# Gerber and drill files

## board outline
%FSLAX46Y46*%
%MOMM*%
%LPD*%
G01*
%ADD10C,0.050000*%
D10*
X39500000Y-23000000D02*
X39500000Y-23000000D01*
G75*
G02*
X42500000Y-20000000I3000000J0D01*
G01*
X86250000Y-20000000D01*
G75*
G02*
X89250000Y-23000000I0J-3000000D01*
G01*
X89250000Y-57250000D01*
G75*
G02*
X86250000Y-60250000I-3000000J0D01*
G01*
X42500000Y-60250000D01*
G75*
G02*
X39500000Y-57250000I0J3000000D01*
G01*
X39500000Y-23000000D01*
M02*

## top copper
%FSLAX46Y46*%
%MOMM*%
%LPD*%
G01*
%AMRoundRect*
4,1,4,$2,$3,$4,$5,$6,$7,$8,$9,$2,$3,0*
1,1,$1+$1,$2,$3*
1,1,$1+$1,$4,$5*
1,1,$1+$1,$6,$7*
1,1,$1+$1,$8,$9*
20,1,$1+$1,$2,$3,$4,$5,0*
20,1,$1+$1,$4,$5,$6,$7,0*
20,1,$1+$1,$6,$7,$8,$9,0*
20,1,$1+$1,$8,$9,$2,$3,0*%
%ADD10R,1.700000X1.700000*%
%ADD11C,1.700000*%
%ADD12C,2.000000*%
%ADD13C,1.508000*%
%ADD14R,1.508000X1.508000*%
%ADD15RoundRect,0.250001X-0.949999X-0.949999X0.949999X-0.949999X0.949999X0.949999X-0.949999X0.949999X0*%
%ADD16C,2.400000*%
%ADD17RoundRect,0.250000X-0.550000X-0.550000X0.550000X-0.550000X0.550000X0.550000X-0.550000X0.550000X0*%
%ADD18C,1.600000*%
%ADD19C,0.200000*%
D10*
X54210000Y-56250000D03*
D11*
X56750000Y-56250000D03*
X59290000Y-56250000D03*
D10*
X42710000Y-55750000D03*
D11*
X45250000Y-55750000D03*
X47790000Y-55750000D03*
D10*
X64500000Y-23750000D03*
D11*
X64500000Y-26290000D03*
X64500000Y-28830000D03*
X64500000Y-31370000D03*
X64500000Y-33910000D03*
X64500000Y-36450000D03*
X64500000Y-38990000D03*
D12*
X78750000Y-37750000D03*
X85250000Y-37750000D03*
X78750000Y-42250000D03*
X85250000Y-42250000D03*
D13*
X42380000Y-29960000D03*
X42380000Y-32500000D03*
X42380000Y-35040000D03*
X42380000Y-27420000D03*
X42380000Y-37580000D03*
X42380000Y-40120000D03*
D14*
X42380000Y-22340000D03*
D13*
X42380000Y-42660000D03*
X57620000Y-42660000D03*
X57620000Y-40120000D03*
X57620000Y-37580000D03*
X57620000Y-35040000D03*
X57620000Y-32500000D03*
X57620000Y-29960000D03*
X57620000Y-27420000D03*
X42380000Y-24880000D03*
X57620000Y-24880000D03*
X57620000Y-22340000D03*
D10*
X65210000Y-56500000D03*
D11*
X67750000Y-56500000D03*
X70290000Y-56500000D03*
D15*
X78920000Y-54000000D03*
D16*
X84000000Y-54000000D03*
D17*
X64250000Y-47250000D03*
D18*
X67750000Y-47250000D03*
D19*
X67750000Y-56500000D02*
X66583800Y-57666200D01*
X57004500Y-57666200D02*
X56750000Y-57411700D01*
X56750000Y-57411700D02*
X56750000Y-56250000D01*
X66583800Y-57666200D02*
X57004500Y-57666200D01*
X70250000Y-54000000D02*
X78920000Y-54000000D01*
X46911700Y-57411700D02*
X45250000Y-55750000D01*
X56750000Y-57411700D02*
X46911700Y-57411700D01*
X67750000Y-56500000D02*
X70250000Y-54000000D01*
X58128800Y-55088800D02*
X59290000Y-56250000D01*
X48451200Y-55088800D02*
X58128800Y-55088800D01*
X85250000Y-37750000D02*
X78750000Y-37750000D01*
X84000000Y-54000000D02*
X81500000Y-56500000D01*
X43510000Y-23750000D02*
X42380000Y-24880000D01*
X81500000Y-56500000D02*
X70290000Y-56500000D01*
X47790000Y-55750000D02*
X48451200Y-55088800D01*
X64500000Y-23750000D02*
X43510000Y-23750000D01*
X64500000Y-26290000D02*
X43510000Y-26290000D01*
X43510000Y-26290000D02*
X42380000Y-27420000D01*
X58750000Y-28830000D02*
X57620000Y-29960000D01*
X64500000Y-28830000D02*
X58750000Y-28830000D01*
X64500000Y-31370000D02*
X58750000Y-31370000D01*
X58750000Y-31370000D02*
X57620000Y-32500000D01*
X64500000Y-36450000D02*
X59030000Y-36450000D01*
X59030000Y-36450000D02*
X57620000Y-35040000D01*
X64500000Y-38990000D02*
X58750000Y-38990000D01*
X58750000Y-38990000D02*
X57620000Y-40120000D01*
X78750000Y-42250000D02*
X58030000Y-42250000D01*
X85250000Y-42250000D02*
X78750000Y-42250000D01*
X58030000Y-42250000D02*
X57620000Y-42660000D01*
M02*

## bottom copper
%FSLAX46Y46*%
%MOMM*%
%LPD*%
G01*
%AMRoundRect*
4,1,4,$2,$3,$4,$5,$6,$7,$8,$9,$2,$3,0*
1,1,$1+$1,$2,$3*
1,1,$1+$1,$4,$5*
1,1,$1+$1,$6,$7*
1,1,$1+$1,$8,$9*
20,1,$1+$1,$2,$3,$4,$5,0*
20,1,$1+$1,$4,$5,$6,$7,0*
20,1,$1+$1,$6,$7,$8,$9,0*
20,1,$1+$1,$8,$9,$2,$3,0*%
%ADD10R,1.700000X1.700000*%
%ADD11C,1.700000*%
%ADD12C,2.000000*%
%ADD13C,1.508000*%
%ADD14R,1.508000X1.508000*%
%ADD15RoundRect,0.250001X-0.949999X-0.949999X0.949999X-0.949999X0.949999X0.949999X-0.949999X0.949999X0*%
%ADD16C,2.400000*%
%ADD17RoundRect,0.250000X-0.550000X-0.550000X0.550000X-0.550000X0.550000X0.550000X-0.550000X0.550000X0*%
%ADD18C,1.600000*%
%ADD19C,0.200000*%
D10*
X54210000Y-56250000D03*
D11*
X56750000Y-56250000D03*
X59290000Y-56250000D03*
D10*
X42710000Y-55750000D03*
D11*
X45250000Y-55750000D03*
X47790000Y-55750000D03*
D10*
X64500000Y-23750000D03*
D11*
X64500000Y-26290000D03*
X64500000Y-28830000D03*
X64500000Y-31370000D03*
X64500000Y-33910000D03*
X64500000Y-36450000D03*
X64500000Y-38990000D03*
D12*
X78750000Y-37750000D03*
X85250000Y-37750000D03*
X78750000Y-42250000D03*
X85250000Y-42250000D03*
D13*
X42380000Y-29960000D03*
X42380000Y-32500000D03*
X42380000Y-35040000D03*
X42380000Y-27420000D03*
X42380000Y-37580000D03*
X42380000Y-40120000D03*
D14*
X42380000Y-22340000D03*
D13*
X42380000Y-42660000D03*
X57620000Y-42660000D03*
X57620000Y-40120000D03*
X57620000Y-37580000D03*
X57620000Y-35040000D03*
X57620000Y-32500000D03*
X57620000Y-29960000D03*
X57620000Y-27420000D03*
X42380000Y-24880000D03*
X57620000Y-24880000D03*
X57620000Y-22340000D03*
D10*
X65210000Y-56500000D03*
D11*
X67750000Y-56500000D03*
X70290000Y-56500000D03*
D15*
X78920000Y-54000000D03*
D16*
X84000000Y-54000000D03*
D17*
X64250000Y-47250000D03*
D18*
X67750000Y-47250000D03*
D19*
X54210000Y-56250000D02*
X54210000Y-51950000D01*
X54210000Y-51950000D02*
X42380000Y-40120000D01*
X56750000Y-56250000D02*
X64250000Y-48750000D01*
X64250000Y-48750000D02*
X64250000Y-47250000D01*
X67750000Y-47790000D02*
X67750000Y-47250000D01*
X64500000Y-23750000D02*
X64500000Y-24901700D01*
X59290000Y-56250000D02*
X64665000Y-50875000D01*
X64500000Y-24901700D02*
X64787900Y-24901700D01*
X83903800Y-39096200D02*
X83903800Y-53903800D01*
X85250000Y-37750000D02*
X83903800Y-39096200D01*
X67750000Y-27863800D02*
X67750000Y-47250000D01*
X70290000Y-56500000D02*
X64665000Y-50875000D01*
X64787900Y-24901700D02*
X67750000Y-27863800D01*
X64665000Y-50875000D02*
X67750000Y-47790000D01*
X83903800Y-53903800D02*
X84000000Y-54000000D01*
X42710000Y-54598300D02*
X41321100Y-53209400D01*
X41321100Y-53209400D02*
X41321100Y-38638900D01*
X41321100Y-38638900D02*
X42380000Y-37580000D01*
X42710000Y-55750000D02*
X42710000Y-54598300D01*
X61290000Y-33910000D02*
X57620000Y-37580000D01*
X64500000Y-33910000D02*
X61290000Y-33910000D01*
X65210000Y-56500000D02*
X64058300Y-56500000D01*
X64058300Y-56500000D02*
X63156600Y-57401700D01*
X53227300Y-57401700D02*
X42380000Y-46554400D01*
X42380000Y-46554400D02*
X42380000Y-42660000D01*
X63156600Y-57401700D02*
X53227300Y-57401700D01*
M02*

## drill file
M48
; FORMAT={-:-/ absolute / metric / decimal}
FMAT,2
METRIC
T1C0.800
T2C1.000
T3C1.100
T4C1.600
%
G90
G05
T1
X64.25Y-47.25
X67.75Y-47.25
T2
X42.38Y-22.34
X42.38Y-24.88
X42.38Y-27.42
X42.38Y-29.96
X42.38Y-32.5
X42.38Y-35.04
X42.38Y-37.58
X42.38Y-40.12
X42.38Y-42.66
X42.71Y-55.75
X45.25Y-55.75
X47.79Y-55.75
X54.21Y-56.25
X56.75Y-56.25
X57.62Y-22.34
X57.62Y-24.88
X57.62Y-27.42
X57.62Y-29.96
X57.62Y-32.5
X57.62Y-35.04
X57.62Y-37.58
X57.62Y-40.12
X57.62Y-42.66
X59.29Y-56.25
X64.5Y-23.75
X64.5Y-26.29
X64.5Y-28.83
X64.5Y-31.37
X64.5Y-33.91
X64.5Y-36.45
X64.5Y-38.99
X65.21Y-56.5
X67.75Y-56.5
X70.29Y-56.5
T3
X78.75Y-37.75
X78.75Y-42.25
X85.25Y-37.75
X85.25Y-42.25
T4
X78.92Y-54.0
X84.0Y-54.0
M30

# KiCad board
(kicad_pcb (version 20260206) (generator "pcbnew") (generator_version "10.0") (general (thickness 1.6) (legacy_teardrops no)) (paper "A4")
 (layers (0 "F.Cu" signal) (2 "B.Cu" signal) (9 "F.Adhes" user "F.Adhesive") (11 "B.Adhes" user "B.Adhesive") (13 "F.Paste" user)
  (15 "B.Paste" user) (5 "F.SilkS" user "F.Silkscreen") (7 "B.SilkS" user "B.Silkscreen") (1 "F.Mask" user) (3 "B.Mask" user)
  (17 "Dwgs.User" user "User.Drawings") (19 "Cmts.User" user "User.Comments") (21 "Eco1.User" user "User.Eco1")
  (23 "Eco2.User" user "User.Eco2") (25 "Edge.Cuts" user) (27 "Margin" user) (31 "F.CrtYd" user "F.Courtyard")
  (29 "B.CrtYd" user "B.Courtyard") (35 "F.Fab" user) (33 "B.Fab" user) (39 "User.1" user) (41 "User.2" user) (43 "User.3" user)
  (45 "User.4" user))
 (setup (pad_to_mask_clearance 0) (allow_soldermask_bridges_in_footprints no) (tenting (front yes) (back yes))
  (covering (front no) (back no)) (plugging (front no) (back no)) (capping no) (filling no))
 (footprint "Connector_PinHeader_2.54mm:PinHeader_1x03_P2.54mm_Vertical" (layer "F.Cu") (at 54.21 56.25 90)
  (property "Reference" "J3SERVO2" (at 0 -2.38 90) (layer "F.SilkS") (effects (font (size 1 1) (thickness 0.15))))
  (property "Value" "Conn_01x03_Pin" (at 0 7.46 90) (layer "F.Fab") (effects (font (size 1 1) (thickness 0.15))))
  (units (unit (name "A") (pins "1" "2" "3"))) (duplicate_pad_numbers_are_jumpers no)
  (pad "1" thru_hole rect (at 0 0 90) (size 1.7 1.7) (drill 1) (layers "*.Cu" "*.Mask") (remove_unused_layers no)
   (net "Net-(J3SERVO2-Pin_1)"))
  (pad "2" thru_hole circle (at 0 2.54 90) (size 1.7 1.7) (drill 1) (layers "*.Cu" "*.Mask") (remove_unused_layers no)
   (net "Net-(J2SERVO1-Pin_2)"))
  (pad "3" thru_hole circle (at 0 5.08 90) (size 1.7 1.7) (drill 1) (layers "*.Cu" "*.Mask") (remove_unused_layers no)
   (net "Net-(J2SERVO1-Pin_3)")))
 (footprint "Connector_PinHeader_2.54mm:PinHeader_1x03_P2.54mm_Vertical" (layer "F.Cu") (at 42.71 55.75 90)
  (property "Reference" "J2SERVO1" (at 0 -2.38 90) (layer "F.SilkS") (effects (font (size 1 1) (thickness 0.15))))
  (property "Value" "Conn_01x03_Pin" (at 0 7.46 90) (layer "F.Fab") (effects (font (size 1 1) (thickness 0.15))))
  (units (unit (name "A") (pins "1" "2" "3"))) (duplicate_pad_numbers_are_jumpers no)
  (pad "1" thru_hole rect (at 0 0 90) (size 1.7 1.7) (drill 1) (layers "*.Cu" "*.Mask") (remove_unused_layers no)
   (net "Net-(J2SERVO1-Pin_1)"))
  (pad "2" thru_hole circle (at 0 2.54 90) (size 1.7 1.7) (drill 1) (layers "*.Cu" "*.Mask") (remove_unused_layers no)
   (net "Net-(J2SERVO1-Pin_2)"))
  (pad "3" thru_hole circle (at 0 5.08 90) (size 1.7 1.7) (drill 1) (layers "*.Cu" "*.Mask") (remove_unused_layers no)
   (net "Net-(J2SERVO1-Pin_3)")))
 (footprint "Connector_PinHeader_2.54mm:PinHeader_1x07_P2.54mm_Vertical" (layer "F.Cu") (at 64.5 23.75)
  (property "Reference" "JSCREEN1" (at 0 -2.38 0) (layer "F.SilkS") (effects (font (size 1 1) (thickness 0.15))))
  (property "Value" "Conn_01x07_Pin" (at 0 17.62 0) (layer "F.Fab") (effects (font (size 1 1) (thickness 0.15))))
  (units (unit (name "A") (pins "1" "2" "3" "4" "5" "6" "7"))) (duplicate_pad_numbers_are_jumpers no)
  (pad "1" thru_hole rect (at 0 0) (size 1.7 1.7) (drill 1) (layers "*.Cu" "*.Mask") (remove_unused_layers no) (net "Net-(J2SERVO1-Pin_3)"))
  (pad "2" thru_hole circle (at 0 2.54) (size 1.7 1.7) (drill 1) (layers "*.Cu" "*.Mask") (remove_unused_layers no)
   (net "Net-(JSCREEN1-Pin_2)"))
  (pad "3" thru_hole circle (at 0 5.08) (size 1.7 1.7) (drill 1) (layers "*.Cu" "*.Mask") (remove_unused_layers no)
   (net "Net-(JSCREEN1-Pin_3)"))
  (pad "4" thru_hole circle (at 0 7.62) (size 1.7 1.7) (drill 1) (layers "*.Cu" "*.Mask") (remove_unused_layers no)
   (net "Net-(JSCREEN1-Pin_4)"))
  (pad "5" thru_hole circle (at 0 10.16) (size 1.7 1.7) (drill 1) (layers "*.Cu" "*.Mask") (remove_unused_layers no)
   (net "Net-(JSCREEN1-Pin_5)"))
  (pad "6" thru_hole circle (at 0 12.7) (size 1.7 1.7) (drill 1) (layers "*.Cu" "*.Mask") (remove_unused_layers no)
   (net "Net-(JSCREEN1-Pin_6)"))
  (pad "7" thru_hole circle (at 0 15.24) (size 1.7 1.7) (drill 1) (layers "*.Cu" "*.Mask") (remove_unused_layers no)
   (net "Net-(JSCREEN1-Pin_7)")))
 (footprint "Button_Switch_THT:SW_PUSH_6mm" (layer "F.Cu") (at 78.75 37.75)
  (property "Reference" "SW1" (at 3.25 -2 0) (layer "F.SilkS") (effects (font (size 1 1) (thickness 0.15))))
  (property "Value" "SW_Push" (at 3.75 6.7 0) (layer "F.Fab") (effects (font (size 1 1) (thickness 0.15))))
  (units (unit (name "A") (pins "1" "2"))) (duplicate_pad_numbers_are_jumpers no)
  (pad "1" thru_hole circle (at 0 0 90) (size 2 2) (drill 1.1) (layers "*.Cu" "*.Mask") (remove_unused_layers no)
   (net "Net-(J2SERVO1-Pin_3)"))
  (pad "1" thru_hole circle (at 6.5 0 90) (size 2 2) (drill 1.1) (layers "*.Cu" "*.Mask") (remove_unused_layers no)
   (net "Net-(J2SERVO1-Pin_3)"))
  (pad "2" thru_hole circle (at 0 4.5 90) (size 2 2) (drill 1.1) (layers "*.Cu" "*.Mask") (remove_unused_layers no) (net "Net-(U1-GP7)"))
  (pad "2" thru_hole circle (at 6.5 4.5 90) (size 2 2) (drill 1.1) (layers "*.Cu" "*.Mask") (remove_unused_layers no) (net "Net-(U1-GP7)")))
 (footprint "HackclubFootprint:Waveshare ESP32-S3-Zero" (layer "F.Cu") (at 50 32.5)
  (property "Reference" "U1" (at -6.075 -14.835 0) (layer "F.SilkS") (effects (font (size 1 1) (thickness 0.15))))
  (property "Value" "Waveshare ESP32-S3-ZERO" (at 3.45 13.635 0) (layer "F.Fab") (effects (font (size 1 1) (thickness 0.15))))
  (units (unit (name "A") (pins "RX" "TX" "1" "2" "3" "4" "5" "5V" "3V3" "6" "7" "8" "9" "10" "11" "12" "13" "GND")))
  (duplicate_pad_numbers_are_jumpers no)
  (pad "1" thru_hole circle (at -7.62 -2.54) (size 1.508 1.508) (drill 1) (layers "*.Cu" "*.Mask") (remove_unused_layers no)
   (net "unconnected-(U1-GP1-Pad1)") (solder_mask_margin 0.102))
  (pad "2" thru_hole circle (at -7.62 0) (size 1.508 1.508) (drill 1) (layers "*.Cu" "*.Mask") (remove_unused_layers no)
   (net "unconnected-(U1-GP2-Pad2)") (solder_mask_margin 0.102))
  (pad "3" thru_hole circle (at -7.62 2.54) (size 1.508 1.508) (drill 1) (layers "*.Cu" "*.Mask") (remove_unused_layers no)
   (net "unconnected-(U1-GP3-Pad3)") (solder_mask_margin 0.102))
  (pad "3V3" thru_hole circle (at -7.62 -5.08) (size 1.508 1.508) (drill 1) (layers "*.Cu" "*.Mask") (remove_unused_layers no)
   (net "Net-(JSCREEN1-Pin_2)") (solder_mask_margin 0.102))
  (pad "4" thru_hole circle (at -7.62 5.08) (size 1.508 1.508) (drill 1) (layers "*.Cu" "*.Mask") (remove_unused_layers no)
   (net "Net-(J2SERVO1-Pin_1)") (solder_mask_margin 0.102))
  (pad "5" thru_hole circle (at -7.62 7.62) (size 1.508 1.508) (drill 1) (layers "*.Cu" "*.Mask") (remove_unused_layers no)
   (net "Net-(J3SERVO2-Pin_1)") (solder_mask_margin 0.102))
  (pad "5V" thru_hole rect (at -7.62 -10.16) (size 1.508 1.508) (drill 1) (layers "*.Cu" "*.Mask") (remove_unused_layers no)
   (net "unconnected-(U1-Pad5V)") (solder_mask_margin 0.102))
  (pad "6" thru_hole circle (at -7.62 10.16) (size 1.508 1.508) (drill 1) (layers "*.Cu" "*.Mask") (remove_unused_layers no)
   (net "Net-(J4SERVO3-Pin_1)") (solder_mask_margin 0.102))
  (pad "7" thru_hole circle (at 7.62 10.16) (size 1.508 1.508) (drill 1) (layers "*.Cu" "*.Mask") (remove_unused_layers no)
   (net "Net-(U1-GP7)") (solder_mask_margin 0.102))
  (pad "8" thru_hole circle (at 7.62 7.62) (size 1.508 1.508) (drill 1) (layers "*.Cu" "*.Mask") (remove_unused_layers no)
   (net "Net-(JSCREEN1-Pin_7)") (solder_mask_margin 0.102))
  (pad "9" thru_hole circle (at 7.62 5.08) (size 1.508 1.508) (drill 1) (layers "*.Cu" "*.Mask") (remove_unused_layers no)
   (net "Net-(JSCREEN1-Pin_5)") (solder_mask_margin 0.102))
  (pad "10" thru_hole circle (at 7.62 2.54) (size 1.508 1.508) (drill 1) (layers "*.Cu" "*.Mask") (remove_unused_layers no)
   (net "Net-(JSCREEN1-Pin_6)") (solder_mask_margin 0.102))
  (pad "11" thru_hole circle (at 7.62 0) (size 1.508 1.508) (drill 1) (layers "*.Cu" "*.Mask") (remove_unused_layers no)
   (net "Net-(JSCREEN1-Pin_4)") (solder_mask_margin 0.102))
  (pad "12" thru_hole circle (at 7.62 -2.54) (size 1.508 1.508) (drill 1) (layers "*.Cu" "*.Mask") (remove_unused_layers no)
   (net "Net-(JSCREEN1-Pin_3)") (solder_mask_margin 0.102))
  (pad "13" thru_hole circle (at 7.62 -5.08) (size 1.508 1.508) (drill 1) (layers "*.Cu" "*.Mask") (remove_unused_layers no)
   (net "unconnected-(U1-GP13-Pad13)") (solder_mask_margin 0.102))
  (pad "GND" thru_hole circle (at -7.62 -7.62) (size 1.508 1.508) (drill 1) (layers "*.Cu" "*.Mask") (remove_unused_layers no)
   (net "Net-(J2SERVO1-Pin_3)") (solder_mask_margin 0.102))
  (pad "RX" thru_hole circle (at 7.62 -7.62) (size 1.508 1.508) (drill 1) (layers "*.Cu" "*.Mask") (remove_unused_layers no)
   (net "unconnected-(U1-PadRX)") (solder_mask_margin 0.102))
  (pad "TX" thru_hole circle (at 7.62 -10.16) (size 1.508 1.508) (drill 1) (layers "*.Cu" "*.Mask") (remove_unused_layers no)
   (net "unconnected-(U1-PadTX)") (solder_mask_margin 0.102)))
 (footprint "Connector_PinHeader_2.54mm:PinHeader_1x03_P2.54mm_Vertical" (layer "F.Cu") (at 65.21 56.5 90)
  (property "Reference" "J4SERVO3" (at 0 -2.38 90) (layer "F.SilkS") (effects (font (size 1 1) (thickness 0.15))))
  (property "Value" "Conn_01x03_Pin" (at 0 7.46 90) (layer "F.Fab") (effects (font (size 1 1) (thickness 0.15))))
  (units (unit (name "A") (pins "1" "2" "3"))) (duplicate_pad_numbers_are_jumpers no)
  (pad "1" thru_hole rect (at 0 0 90) (size 1.7 1.7) (drill 1) (layers "*.Cu" "*.Mask") (remove_unused_layers no)
   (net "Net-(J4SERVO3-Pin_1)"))
  (pad "2" thru_hole circle (at 0 2.54 90) (size 1.7 1.7) (drill 1) (layers "*.Cu" "*.Mask") (remove_unused_layers no)
   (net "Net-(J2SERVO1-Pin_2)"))
  (pad "3" thru_hole circle (at 0 5.08 90) (size 1.7 1.7) (drill 1) (layers "*.Cu" "*.Mask") (remove_unused_layers no)
   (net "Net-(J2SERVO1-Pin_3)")))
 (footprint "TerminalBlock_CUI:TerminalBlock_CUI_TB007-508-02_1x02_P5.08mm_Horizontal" (layer "F.Cu") (at 78.92 54)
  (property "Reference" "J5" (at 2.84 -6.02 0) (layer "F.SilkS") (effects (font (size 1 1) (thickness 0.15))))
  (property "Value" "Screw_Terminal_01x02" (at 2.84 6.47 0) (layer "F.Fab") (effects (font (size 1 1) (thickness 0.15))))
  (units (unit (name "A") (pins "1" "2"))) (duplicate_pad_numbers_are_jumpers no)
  (pad "1" thru_hole roundrect (at 0 0) (size 2.4 2.4) (drill 1.6) (layers "*.Cu" "*.Mask") (remove_unused_layers no)
   (roundrect_rratio 0.104167) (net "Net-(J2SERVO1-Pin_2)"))
  (pad "2" thru_hole circle (at 5.08 0) (size 2.4 2.4) (drill 1.6) (layers "*.Cu" "*.Mask") (remove_unused_layers no)
   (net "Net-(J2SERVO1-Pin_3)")))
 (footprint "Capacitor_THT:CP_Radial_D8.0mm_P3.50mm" (layer "F.Cu") (at 64.25 47.25)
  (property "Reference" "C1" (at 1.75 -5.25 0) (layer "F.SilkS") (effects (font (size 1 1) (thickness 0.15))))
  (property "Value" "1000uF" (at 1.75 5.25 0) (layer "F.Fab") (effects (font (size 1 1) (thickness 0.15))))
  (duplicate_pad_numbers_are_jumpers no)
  (pad "1" thru_hole roundrect (at 0 0) (size 1.6 1.6) (drill 0.8) (layers "*.Cu" "*.Mask") (remove_unused_layers no)
   (roundrect_rratio 0.15625) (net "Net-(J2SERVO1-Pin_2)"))
  (pad "2" thru_hole circle (at 3.5 0) (size 1.6 1.6) (drill 0.8) (layers "*.Cu" "*.Mask") (remove_unused_layers no)
   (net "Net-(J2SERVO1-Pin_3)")))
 (gr_rect (start 39.5 20) (end 89.25 60.25) (radius 3) (stroke (width 0.05) (type solid)) (fill no) (layer "Edge.Cuts"))
 (segment (start 54.21 56.25) (end 54.21 51.95) (width 0.2) (layer "B.Cu") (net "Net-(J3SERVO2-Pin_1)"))
 (segment (start 54.21 51.95) (end 42.38 40.12) (width 0.2) (layer "B.Cu") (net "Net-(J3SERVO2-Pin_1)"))
 (segment (start 67.75 56.5) (end 66.5838 57.6662) (width 0.2) (layer "F.Cu") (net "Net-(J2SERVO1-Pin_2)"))
 (segment (start 57.0045 57.6662) (end 56.75 57.4117) (width 0.2) (layer "F.Cu") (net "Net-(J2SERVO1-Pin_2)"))
 (segment (start 56.75 57.4117) (end 56.75 56.25) (width 0.2) (layer "F.Cu") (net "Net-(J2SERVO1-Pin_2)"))
 (segment (start 66.5838 57.6662) (end 57.0045 57.6662) (width 0.2) (layer "F.Cu") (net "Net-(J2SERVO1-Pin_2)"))
 (segment (start 70.25 54) (end 78.92 54) (width 0.2) (layer "F.Cu") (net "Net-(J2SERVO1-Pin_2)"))
 (segment (start 46.9117 57.4117) (end 45.25 55.75) (width 0.2) (layer "F.Cu") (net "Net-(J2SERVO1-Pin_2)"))
 (segment (start 56.75 57.4117) (end 46.9117 57.4117) (width 0.2) (layer "F.Cu") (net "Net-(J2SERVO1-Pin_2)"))
 (segment (start 67.75 56.5) (end 70.25 54) (width 0.2) (layer "F.Cu") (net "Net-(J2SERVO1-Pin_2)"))
 (segment (start 56.75 56.25) (end 64.25 48.75) (width 0.2) (layer "B.Cu") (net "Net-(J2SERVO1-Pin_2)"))
 (segment (start 64.25 48.75) (end 64.25 47.25) (width 0.2) (layer "B.Cu") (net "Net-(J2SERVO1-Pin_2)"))
 (segment (start 58.1288 55.0888) (end 59.29 56.25) (width 0.2) (layer "F.Cu") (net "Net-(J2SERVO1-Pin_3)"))
 (segment (start 48.4512 55.0888) (end 58.1288 55.0888) (width 0.2) (layer "F.Cu") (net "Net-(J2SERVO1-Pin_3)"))
 (segment (start 85.25 37.75) (end 78.75 37.75) (width 0.2) (layer "F.Cu") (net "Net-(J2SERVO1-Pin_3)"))
 (segment (start 84 54) (end 81.5 56.5) (width 0.2) (layer "F.Cu") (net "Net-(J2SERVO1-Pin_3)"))
 (segment (start 43.51 23.75) (end 42.38 24.88) (width 0.2) (layer "F.Cu") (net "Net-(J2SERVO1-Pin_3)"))
 (segment (start 81.5 56.5) (end 70.29 56.5) (width 0.2) (layer "F.Cu") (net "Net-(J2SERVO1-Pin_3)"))
 (segment (start 47.79 55.75) (end 48.4512 55.0888) (width 0.2) (layer "F.Cu") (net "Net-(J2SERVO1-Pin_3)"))
 (segment (start 64.5 23.75) (end 43.51 23.75) (width 0.2) (layer "F.Cu") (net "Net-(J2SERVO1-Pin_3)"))
 (segment (start 67.75 47.79) (end 67.75 47.25) (width 0.2) (layer "B.Cu") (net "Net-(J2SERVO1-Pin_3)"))
 (segment (start 64.5 23.75) (end 64.5 24.9017) (width 0.2) (layer "B.Cu") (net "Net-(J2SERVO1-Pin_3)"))
 (segment (start 59.29 56.25) (end 64.665 50.875) (width 0.2) (layer "B.Cu") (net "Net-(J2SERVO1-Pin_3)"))
 (segment (start 64.5 24.9017) (end 64.7879 24.9017) (width 0.2) (layer "B.Cu") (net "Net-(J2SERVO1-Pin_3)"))
 (segment (start 83.9038 39.0962) (end 83.9038 53.9038) (width 0.2) (layer "B.Cu") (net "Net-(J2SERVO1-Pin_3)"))
 (segment (start 85.25 37.75) (end 83.9038 39.0962) (width 0.2) (layer "B.Cu") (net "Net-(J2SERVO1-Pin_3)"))
 (segment (start 67.75 27.8638) (end 67.75 47.25) (width 0.2) (layer "B.Cu") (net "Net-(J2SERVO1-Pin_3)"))
 (segment (start 70.29 56.5) (end 64.665 50.875) (width 0.2) (layer "B.Cu") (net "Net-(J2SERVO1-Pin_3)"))
 (segment (start 64.7879 24.9017) (end 67.75 27.8638) (width 0.2) (layer "B.Cu") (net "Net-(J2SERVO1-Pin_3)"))
 (segment (start 64.665 50.875) (end 67.75 47.79) (width 0.2) (layer "B.Cu") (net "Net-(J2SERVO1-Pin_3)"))
 (segment (start 83.9038 53.9038) (end 84 54) (width 0.2) (layer "B.Cu") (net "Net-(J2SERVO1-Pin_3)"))
 (segment (start 42.71 54.5983) (end 41.3211 53.2094) (width 0.2) (layer "B.Cu") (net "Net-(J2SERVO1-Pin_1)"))
 (segment (start 41.3211 53.2094) (end 41.3211 38.6389) (width 0.2) (layer "B.Cu") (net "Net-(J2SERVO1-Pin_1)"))
 (segment (start 41.3211 38.6389) (end 42.38 37.58) (width 0.2) (layer "B.Cu") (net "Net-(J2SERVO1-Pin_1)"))
 (segment (start 42.71 55.75) (end 42.71 54.5983) (width 0.2) (layer "B.Cu") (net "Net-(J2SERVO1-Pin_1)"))
 (segment (start 64.5 26.29) (end 43.51 26.29) (width 0.2) (layer "F.Cu") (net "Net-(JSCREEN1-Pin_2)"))
 (segment (start 43.51 26.29) (end 42.38 27.42) (width 0.2) (layer "F.Cu") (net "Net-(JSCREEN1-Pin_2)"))
 (segment (start 58.75 28.83) (end 57.62 29.96) (width 0.2) (layer "F.Cu") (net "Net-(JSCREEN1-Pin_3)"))
 (segment (start 64.5 28.83) (end 58.75 28.83) (width 0.2) (layer "F.Cu") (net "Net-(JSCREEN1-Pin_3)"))
 (segment (start 64.5 31.37) (end 58.75 31.37) (width 0.2) (layer "F.Cu") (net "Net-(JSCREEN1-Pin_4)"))
 (segment (start 58.75 31.37) (end 57.62 32.5) (width 0.2) (layer "F.Cu") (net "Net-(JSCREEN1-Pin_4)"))
 (segment (start 61.29 33.91) (end 57.62 37.58) (width 0.2) (layer "B.Cu") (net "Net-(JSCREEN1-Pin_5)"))
 (segment (start 64.5 33.91) (end 61.29 33.91) (width 0.2) (layer "B.Cu") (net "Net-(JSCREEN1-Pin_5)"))
 (segment (start 64.5 36.45) (end 59.03 36.45) (width 0.2) (layer "F.Cu") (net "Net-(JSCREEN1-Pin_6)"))
 (segment (start 59.03 36.45) (end 57.62 35.04) (width 0.2) (layer "F.Cu") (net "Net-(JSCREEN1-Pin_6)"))
 (segment (start 64.5 38.99) (end 58.75 38.99) (width 0.2) (layer "F.Cu") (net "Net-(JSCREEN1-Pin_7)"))
 (segment (start 58.75 38.99) (end 57.62 40.12) (width 0.2) (layer "F.Cu") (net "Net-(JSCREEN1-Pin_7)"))
 (segment (start 78.75 42.25) (end 58.03 42.25) (width 0.2) (layer "F.Cu") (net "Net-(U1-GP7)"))
 (segment (start 85.25 42.25) (end 78.75 42.25) (width 0.2) (layer "F.Cu") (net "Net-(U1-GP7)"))
 (segment (start 58.03 42.25) (end 57.62 42.66) (width 0.2) (layer "F.Cu") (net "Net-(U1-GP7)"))
 (segment (start 65.21 56.5) (end 64.0583 56.5) (width 0.2) (layer "B.Cu") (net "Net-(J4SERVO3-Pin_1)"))
 (segment (start 64.0583 56.5) (end 63.1566 57.4017) (width 0.2) (layer "B.Cu") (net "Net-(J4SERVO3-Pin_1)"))
 (segment (start 53.2273 57.4017) (end 42.38 46.5544) (width 0.2) (layer "B.Cu") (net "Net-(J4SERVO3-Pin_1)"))
 (segment (start 42.38 46.5544) (end 42.38 42.66) (width 0.2) (layer "B.Cu") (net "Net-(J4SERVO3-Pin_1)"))
 (segment (start 63.1566 57.4017) (end 53.2273 57.4017) (width 0.2) (layer "B.Cu") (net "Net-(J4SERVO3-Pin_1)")))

